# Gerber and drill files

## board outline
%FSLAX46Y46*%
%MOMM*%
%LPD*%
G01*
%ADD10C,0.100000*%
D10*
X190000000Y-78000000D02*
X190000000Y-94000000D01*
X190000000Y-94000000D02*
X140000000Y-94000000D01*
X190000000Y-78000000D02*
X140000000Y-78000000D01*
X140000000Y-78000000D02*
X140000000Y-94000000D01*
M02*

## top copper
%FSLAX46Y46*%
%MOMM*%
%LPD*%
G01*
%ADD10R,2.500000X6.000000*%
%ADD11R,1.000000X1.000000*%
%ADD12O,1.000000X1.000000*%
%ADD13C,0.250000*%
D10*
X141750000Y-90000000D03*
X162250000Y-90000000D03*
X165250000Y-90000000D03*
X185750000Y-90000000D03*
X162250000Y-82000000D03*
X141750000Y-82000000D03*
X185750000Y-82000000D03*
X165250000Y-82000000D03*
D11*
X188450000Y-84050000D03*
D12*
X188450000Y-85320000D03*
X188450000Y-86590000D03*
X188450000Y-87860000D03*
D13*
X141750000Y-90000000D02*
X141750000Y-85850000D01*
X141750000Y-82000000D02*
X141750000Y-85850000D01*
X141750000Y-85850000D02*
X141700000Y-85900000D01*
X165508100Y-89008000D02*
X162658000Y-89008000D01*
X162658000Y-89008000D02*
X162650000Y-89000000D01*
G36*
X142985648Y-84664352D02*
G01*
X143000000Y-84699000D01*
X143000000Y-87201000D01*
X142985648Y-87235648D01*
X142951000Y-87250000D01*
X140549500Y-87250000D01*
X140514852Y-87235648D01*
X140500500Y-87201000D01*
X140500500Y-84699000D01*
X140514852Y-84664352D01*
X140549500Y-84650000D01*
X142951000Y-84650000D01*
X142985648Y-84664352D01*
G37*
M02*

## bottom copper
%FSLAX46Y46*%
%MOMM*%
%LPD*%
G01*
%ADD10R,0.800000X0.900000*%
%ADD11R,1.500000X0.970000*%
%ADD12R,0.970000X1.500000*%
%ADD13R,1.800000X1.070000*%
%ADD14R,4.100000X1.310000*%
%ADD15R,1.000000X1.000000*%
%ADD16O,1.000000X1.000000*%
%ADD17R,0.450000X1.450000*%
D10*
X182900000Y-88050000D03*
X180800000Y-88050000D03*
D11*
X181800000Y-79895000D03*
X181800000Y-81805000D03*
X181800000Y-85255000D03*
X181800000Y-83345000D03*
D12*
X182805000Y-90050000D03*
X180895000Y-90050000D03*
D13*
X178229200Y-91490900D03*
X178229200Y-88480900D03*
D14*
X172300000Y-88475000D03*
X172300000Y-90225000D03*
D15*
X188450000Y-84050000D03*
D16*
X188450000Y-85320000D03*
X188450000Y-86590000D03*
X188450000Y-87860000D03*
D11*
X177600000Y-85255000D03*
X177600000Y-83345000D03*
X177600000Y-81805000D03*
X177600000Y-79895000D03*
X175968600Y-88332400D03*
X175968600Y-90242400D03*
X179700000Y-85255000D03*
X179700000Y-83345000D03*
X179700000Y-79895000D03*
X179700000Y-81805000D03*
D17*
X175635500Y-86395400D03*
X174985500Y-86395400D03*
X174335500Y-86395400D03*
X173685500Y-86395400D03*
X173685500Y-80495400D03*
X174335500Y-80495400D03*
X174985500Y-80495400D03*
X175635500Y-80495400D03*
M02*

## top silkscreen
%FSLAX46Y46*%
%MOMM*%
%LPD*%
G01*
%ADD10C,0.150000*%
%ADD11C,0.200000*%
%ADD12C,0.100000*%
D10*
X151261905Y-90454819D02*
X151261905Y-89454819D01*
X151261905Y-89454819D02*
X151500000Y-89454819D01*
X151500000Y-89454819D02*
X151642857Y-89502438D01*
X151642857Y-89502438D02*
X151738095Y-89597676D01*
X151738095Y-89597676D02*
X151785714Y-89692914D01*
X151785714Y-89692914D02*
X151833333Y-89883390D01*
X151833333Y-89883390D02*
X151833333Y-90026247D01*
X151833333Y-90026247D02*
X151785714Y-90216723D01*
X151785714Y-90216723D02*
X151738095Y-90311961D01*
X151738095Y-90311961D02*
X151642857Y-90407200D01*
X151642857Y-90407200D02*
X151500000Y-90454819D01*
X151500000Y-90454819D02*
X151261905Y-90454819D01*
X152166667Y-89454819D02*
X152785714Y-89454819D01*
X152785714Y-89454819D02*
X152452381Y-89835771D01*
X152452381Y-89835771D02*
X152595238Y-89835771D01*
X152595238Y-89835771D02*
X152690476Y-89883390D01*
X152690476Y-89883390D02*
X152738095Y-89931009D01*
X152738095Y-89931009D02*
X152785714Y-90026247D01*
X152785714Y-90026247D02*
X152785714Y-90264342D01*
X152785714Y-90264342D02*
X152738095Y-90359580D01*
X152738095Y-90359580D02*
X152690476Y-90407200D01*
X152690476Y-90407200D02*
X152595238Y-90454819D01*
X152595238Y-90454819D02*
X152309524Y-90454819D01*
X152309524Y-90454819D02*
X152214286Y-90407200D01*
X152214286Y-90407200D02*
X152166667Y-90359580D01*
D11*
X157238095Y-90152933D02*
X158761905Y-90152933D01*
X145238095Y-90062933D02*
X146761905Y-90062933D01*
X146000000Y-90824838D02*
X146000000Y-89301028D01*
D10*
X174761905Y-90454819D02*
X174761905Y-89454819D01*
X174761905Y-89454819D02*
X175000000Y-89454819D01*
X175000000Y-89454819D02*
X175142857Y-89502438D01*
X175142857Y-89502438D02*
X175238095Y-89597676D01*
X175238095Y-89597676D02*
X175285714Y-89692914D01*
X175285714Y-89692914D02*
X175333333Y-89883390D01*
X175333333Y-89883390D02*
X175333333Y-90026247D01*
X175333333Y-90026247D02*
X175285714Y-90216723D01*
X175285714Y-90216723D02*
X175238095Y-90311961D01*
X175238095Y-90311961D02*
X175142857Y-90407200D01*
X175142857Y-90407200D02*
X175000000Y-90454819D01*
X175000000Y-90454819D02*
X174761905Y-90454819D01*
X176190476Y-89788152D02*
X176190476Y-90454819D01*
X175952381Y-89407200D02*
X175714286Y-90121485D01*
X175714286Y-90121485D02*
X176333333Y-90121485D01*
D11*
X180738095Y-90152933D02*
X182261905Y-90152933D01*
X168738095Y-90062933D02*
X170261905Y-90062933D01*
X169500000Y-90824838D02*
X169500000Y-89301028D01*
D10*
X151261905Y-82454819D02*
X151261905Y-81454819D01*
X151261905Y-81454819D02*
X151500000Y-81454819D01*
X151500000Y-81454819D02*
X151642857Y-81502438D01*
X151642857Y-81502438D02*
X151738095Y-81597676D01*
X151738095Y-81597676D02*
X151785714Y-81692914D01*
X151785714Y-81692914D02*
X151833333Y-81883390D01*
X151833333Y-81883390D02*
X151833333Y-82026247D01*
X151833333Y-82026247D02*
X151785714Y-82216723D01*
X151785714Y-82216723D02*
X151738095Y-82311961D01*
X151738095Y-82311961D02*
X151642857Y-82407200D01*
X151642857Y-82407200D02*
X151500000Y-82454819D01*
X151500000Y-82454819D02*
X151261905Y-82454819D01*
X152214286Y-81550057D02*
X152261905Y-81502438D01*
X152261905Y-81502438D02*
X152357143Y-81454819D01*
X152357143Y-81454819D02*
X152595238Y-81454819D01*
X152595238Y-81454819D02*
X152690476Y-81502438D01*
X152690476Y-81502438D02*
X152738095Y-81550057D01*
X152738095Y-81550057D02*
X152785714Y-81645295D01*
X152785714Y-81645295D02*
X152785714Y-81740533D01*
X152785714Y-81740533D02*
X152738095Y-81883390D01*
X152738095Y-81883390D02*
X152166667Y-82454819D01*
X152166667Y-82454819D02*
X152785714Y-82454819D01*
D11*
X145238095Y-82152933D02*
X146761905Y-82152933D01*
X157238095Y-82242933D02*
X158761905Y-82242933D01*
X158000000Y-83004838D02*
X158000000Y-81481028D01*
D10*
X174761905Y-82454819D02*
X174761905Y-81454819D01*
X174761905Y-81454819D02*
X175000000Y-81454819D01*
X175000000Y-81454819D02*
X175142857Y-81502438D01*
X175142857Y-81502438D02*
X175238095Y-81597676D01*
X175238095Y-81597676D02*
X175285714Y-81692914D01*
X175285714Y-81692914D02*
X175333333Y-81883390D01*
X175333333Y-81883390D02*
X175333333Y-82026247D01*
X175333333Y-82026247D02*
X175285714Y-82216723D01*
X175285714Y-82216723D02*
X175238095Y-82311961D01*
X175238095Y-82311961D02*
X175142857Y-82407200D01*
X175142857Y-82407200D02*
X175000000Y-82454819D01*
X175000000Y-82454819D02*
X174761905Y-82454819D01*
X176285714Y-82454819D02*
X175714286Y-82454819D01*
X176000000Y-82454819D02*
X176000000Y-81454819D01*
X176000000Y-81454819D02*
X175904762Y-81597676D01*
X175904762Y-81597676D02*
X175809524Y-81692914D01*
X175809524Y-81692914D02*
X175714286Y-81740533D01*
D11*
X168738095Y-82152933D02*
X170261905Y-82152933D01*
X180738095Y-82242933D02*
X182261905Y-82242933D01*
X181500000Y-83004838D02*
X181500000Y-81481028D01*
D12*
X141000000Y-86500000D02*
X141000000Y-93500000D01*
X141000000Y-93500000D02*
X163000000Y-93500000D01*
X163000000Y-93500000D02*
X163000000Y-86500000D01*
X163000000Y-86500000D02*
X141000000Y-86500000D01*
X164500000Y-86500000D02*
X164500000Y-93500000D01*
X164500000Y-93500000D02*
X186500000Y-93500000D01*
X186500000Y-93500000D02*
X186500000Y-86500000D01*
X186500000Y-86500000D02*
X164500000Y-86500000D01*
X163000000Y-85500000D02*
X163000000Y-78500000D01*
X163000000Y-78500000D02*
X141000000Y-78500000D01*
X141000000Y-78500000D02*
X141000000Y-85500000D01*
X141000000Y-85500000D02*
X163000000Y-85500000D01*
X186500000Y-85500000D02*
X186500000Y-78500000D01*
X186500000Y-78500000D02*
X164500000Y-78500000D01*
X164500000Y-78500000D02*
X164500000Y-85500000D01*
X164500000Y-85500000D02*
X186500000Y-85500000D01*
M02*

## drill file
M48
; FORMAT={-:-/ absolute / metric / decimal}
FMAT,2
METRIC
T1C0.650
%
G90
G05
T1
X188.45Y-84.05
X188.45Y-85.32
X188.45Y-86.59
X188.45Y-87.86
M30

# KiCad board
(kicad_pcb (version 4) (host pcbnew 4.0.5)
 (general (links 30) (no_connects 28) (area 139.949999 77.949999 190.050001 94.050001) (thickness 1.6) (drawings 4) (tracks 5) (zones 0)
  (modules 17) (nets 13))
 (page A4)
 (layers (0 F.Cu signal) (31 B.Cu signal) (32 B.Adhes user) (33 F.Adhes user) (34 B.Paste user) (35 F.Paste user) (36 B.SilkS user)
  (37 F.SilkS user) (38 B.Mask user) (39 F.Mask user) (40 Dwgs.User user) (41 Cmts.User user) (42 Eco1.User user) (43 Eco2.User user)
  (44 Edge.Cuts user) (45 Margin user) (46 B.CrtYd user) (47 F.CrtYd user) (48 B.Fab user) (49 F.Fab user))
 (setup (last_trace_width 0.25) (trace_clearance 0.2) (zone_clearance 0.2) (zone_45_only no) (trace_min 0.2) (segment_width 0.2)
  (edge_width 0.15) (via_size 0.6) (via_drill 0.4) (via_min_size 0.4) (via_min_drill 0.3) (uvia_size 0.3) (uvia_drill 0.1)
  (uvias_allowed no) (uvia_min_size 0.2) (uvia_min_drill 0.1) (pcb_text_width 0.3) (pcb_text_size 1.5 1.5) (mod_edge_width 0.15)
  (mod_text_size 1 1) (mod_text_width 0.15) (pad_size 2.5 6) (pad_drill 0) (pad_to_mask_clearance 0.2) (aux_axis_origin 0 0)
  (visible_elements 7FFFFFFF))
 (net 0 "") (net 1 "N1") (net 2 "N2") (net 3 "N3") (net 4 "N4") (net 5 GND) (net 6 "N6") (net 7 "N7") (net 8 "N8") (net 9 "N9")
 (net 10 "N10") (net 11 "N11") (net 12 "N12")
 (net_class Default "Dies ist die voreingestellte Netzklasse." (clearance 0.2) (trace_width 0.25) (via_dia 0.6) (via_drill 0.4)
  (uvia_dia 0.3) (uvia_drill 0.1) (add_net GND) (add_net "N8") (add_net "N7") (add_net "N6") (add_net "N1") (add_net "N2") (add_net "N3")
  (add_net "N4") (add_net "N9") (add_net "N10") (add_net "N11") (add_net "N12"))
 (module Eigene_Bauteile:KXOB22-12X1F (layer F.Cu) (at 152 90)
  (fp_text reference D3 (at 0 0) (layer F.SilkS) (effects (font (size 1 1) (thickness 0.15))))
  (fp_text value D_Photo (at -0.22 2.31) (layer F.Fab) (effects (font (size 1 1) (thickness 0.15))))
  (fp_line (start -11 -3.5) (end -11 3.5) (layer F.SilkS) (width 0.1))
  (fp_line (start -11 3.5) (end 11 3.5) (layer F.SilkS) (width 0.1))
  (fp_line (start 11 3.5) (end 11 -3.5) (layer F.SilkS) (width 0.1))
  (fp_line (start 11 -3.5) (end -11 -3.5) (layer F.SilkS) (width 0.1))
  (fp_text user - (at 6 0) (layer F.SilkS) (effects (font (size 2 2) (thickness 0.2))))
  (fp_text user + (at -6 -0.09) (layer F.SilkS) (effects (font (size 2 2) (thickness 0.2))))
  (pad 1 smd rect (at -10.25 0) (size 2.5 6) (layers F.Cu F.Paste F.Mask) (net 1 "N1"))
  (pad 2 smd rect (at 10.25 0) (size 2.5 6) (layers F.Cu F.Paste F.Mask) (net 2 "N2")))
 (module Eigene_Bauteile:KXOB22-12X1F (layer F.Cu) (at 175.5 90)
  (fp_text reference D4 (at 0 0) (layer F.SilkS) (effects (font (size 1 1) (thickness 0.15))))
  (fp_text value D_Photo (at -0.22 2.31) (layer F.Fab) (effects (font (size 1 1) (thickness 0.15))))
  (fp_line (start -11 -3.5) (end -11 3.5) (layer F.SilkS) (width 0.1))
  (fp_line (start -11 3.5) (end 11 3.5) (layer F.SilkS) (width 0.1))
  (fp_line (start 11 3.5) (end 11 -3.5) (layer F.SilkS) (width 0.1))
  (fp_line (start 11 -3.5) (end -11 -3.5) (layer F.SilkS) (width 0.1))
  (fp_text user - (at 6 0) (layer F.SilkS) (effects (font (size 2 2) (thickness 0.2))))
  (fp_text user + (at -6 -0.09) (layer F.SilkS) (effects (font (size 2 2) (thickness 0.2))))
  (pad 1 smd rect (at -10.25 0) (size 2.5 6) (layers F.Cu F.Paste F.Mask) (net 2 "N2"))
  (pad 2 smd rect (at 10.25 0) (size 2.5 6) (layers F.Cu F.Paste F.Mask) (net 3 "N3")))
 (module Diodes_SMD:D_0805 (layer B.Cu) (at 181.85 88.05 180)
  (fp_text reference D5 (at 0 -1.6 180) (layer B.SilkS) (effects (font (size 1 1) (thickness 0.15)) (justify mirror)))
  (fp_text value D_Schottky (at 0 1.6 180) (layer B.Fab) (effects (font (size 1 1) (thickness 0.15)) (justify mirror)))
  (pad 1 smd rect (at -1.05 0 180) (size 0.8 0.9) (layers B.Cu B.Paste B.Mask) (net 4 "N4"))
  (pad 2 smd rect (at 1.05 0 180) (size 0.8 0.9) (layers B.Cu B.Paste B.Mask) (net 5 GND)))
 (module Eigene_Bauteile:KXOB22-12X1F (layer F.Cu) (at 152 82 180)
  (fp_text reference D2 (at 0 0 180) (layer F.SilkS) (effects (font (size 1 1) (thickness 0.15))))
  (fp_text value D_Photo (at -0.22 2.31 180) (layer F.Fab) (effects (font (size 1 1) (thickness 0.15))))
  (fp_line (start -11 -3.5) (end -11 3.5) (layer F.SilkS) (width 0.1))
  (fp_line (start -11 3.5) (end 11 3.5) (layer F.SilkS) (width 0.1))
  (fp_line (start 11 3.5) (end 11 -3.5) (layer F.SilkS) (width 0.1))
  (fp_line (start 11 -3.5) (end -11 -3.5) (layer F.SilkS) (width 0.1))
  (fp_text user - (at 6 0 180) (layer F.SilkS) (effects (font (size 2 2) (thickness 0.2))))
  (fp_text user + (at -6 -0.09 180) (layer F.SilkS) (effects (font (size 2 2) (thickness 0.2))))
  (pad 1 smd rect (at -10.25 0 180) (size 2.5 6) (layers F.Cu F.Paste F.Mask) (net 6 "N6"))
  (pad 2 smd rect (at 10.25 0 180) (size 2.5 6) (layers F.Cu F.Paste F.Mask) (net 1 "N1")))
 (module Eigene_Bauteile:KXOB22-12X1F (layer F.Cu) (at 175.5 82 180)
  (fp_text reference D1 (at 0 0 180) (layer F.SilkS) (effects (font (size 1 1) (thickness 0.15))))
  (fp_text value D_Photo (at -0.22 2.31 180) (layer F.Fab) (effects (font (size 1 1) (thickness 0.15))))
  (fp_line (start -11 -3.5) (end -11 3.5) (layer F.SilkS) (width 0.1))
  (fp_line (start -11 3.5) (end 11 3.5) (layer F.SilkS) (width 0.1))
  (fp_line (start 11 3.5) (end 11 -3.5) (layer F.SilkS) (width 0.1))
  (fp_line (start 11 -3.5) (end -11 -3.5) (layer F.SilkS) (width 0.1))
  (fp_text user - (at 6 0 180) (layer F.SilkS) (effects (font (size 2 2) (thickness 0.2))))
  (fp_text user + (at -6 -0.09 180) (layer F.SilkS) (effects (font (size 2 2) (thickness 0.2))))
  (pad 1 smd rect (at -10.25 0 180) (size 2.5 6) (layers F.Cu F.Paste F.Mask) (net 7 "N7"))
  (pad 2 smd rect (at 10.25 0 180) (size 2.5 6) (layers F.Cu F.Paste F.Mask) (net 6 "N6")))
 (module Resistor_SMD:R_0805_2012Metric (layer B.Cu) (at 181.8 80.85 270)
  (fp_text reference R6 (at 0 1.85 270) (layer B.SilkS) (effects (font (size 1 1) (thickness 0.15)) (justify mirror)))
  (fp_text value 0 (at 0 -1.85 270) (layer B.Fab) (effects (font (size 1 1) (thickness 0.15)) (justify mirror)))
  (pad 1 smd rect (at -0.955 0 270) (size 0.97 1.5) (layers B.Cu B.Paste B.Mask) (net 5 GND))
  (pad 2 smd rect (at 0.955 0 270) (size 0.97 1.5) (layers B.Cu B.Paste B.Mask) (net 3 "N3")))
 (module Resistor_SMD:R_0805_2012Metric (layer B.Cu) (at 181.8 84.3 90)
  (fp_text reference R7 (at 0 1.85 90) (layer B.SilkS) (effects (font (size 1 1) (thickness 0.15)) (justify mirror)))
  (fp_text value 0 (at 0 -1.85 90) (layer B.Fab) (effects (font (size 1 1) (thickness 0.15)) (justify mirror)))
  (pad 1 smd rect (at -0.955 0 90) (size 0.97 1.5) (layers B.Cu B.Paste B.Mask) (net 4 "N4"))
  (pad 2 smd rect (at 0.955 0 90) (size 0.97 1.5) (layers B.Cu B.Paste B.Mask) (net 7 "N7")))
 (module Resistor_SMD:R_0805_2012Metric (layer B.Cu) (at 181.85 90.05 180)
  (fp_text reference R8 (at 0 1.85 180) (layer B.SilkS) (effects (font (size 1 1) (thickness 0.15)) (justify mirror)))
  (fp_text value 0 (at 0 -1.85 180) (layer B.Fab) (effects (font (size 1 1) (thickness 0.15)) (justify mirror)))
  (pad 1 smd rect (at -0.955 0 180) (size 0.97 1.5) (layers B.Cu B.Paste B.Mask) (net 3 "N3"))
  (pad 2 smd rect (at 0.955 0 180) (size 0.97 1.5) (layers B.Cu B.Paste B.Mask) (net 5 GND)))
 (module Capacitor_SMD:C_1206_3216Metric (layer B.Cu) (at 178.2292 89.9859 90)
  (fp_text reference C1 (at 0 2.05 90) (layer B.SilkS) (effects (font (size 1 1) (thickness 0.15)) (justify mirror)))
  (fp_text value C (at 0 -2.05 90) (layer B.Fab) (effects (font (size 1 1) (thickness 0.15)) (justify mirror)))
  (pad 1 smd rect (at -1.505 0 90) (size 1.07 1.8) (layers B.Cu B.Paste B.Mask) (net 5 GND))
  (pad 2 smd rect (at 1.505 0 90) (size 1.07 1.8) (layers B.Cu B.Paste B.Mask) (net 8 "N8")))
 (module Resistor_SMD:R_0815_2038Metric (layer B.Cu) (at 172.3 89.35 270)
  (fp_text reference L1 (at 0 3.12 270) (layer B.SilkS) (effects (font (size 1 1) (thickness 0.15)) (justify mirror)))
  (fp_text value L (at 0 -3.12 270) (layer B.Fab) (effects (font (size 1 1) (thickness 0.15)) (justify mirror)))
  (pad 1 smd rect (at -0.875 0 270) (size 1.31 4.1) (layers B.Cu B.Paste B.Mask) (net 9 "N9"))
  (pad 2 smd rect (at 0.875 0 270) (size 1.31 4.1) (layers B.Cu B.Paste B.Mask) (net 7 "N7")))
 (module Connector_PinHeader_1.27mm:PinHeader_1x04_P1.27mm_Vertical (layer B.Cu) (at 188.45 84.05 180)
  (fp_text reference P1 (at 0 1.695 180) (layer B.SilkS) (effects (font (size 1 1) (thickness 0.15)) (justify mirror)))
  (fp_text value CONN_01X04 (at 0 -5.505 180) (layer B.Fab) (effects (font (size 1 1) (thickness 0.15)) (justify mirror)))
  (pad 1 thru_hole rect (at 0 0 180) (size 1 1) (drill 0.65) (layers *.Cu *.Mask) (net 4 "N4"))
  (pad 2 thru_hole oval (at 0 -1.27 180) (size 1 1) (drill 0.65) (layers *.Cu *.Mask) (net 5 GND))
  (pad 3 thru_hole oval (at 0 -2.54 180) (size 1 1) (drill 0.65) (layers *.Cu *.Mask) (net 3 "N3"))
  (pad 4 thru_hole oval (at 0 -3.81 180) (size 1 1) (drill 0.65) (layers *.Cu *.Mask) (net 5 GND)))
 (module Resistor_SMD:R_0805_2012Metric (layer B.Cu) (at 177.6 84.3 90)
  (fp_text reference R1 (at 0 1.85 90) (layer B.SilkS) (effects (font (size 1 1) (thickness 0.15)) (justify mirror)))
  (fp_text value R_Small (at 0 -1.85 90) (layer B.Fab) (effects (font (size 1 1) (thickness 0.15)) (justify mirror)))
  (pad 1 smd rect (at -0.955 0 90) (size 0.97 1.5) (layers B.Cu B.Paste B.Mask) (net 8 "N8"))
  (pad 2 smd rect (at 0.955 0 90) (size 0.97 1.5) (layers B.Cu B.Paste B.Mask) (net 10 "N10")))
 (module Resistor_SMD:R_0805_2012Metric (layer B.Cu) (at 177.6 80.85 90)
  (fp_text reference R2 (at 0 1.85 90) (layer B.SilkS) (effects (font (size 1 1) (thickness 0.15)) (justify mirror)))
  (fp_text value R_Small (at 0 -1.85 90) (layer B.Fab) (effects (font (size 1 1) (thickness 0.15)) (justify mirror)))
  (pad 1 smd rect (at -0.955 0 90) (size 0.97 1.5) (layers B.Cu B.Paste B.Mask) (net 4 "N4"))
  (pad 2 smd rect (at 0.955 0 90) (size 0.97 1.5) (layers B.Cu B.Paste B.Mask) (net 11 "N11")))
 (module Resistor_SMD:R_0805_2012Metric (layer B.Cu) (at 175.9686 89.2874 270)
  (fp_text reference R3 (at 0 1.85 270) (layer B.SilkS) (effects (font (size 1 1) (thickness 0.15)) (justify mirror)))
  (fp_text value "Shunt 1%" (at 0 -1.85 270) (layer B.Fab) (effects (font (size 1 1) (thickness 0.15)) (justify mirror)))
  (pad 1 smd rect (at -0.955 0 270) (size 0.97 1.5) (layers B.Cu B.Paste B.Mask) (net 8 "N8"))
  (pad 2 smd rect (at 0.955 0 270) (size 0.97 1.5) (layers B.Cu B.Paste B.Mask) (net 4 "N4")))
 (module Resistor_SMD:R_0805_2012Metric (layer B.Cu) (at 179.7 84.3 90)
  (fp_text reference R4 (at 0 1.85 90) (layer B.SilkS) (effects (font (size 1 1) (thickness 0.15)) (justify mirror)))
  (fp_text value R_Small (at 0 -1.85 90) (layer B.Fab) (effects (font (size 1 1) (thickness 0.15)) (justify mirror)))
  (pad 1 smd rect (at -0.955 0 90) (size 0.97 1.5) (layers B.Cu B.Paste B.Mask) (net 4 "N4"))
  (pad 2 smd rect (at 0.955 0 90) (size 0.97 1.5) (layers B.Cu B.Paste B.Mask) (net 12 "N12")))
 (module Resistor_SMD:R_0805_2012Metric (layer B.Cu) (at 179.7 80.85 270)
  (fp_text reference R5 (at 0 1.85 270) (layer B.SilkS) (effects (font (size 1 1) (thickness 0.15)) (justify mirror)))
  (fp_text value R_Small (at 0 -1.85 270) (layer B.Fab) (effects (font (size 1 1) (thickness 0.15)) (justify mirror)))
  (pad 1 smd rect (at -0.955 0 270) (size 0.97 1.5) (layers B.Cu B.Paste B.Mask) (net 12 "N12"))
  (pad 2 smd rect (at 0.955 0 270) (size 0.97 1.5) (layers B.Cu B.Paste B.Mask) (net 5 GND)))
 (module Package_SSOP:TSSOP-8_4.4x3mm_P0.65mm (layer B.Cu) (at 174.6605 83.4454 90)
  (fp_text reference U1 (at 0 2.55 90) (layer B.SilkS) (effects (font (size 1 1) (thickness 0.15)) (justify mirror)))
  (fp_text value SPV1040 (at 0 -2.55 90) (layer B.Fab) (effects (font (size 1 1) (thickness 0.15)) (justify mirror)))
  (pad 1 smd rect (at -2.95 0.975 90) (size 1.45 0.45) (layers B.Cu B.Paste B.Mask) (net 7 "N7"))
  (pad 2 smd rect (at -2.95 0.325 90) (size 1.45 0.45) (layers B.Cu B.Paste B.Mask) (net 5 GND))
  (pad 3 smd rect (at -2.95 -0.325 90) (size 1.45 0.45) (layers B.Cu B.Paste B.Mask) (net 9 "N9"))
  (pad 4 smd rect (at -2.95 -0.975 90) (size 1.45 0.45) (layers B.Cu B.Paste B.Mask) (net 8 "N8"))
  (pad 5 smd rect (at 2.95 -0.975 90) (size 1.45 0.45) (layers B.Cu B.Paste B.Mask) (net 12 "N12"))
  (pad 6 smd rect (at 2.95 -0.325 90) (size 1.45 0.45) (layers B.Cu B.Paste B.Mask) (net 11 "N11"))
  (pad 7 smd rect (at 2.95 0.325 90) (size 1.45 0.45) (layers B.Cu B.Paste B.Mask) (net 10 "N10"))
  (pad 8 smd rect (at 2.95 0.975 90) (size 1.45 0.45) (layers B.Cu B.Paste B.Mask) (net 7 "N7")))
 (gr_line (start 190 78) (end 190 94) (angle 90) (layer Edge.Cuts) (width 0.1))
 (gr_line (start 190 94) (end 140 94) (angle 90) (layer Edge.Cuts) (width 0.1))
 (gr_line (start 190 78) (end 140 78) (angle 90) (layer Edge.Cuts) (width 0.1))
 (gr_line (start 140 78) (end 140 94) (angle 90) (layer Edge.Cuts) (width 0.1))
 (segment (start 141.75 90) (end 141.75 85.85) (width 0.25) (layer F.Cu) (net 1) (status 400000))
 (segment (start 141.75 82) (end 141.75 85.85) (width 0.25) (layer F.Cu) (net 1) (status 400000))
 (segment (start 141.75 85.85) (end 141.7 85.9) (width 0.25) (layer F.Cu) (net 1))
 (segment (start 165.5081 89.008) (end 162.658 89.008) (width 0.25) (layer F.Cu) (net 2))
 (segment (start 162.658 89.008) (end 162.65 89) (width 0.25) (layer F.Cu) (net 2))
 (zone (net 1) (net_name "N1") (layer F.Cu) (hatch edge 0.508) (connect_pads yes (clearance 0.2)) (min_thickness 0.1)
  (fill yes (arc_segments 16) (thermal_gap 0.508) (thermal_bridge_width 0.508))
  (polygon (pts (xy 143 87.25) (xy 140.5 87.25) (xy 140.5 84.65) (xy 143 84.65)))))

